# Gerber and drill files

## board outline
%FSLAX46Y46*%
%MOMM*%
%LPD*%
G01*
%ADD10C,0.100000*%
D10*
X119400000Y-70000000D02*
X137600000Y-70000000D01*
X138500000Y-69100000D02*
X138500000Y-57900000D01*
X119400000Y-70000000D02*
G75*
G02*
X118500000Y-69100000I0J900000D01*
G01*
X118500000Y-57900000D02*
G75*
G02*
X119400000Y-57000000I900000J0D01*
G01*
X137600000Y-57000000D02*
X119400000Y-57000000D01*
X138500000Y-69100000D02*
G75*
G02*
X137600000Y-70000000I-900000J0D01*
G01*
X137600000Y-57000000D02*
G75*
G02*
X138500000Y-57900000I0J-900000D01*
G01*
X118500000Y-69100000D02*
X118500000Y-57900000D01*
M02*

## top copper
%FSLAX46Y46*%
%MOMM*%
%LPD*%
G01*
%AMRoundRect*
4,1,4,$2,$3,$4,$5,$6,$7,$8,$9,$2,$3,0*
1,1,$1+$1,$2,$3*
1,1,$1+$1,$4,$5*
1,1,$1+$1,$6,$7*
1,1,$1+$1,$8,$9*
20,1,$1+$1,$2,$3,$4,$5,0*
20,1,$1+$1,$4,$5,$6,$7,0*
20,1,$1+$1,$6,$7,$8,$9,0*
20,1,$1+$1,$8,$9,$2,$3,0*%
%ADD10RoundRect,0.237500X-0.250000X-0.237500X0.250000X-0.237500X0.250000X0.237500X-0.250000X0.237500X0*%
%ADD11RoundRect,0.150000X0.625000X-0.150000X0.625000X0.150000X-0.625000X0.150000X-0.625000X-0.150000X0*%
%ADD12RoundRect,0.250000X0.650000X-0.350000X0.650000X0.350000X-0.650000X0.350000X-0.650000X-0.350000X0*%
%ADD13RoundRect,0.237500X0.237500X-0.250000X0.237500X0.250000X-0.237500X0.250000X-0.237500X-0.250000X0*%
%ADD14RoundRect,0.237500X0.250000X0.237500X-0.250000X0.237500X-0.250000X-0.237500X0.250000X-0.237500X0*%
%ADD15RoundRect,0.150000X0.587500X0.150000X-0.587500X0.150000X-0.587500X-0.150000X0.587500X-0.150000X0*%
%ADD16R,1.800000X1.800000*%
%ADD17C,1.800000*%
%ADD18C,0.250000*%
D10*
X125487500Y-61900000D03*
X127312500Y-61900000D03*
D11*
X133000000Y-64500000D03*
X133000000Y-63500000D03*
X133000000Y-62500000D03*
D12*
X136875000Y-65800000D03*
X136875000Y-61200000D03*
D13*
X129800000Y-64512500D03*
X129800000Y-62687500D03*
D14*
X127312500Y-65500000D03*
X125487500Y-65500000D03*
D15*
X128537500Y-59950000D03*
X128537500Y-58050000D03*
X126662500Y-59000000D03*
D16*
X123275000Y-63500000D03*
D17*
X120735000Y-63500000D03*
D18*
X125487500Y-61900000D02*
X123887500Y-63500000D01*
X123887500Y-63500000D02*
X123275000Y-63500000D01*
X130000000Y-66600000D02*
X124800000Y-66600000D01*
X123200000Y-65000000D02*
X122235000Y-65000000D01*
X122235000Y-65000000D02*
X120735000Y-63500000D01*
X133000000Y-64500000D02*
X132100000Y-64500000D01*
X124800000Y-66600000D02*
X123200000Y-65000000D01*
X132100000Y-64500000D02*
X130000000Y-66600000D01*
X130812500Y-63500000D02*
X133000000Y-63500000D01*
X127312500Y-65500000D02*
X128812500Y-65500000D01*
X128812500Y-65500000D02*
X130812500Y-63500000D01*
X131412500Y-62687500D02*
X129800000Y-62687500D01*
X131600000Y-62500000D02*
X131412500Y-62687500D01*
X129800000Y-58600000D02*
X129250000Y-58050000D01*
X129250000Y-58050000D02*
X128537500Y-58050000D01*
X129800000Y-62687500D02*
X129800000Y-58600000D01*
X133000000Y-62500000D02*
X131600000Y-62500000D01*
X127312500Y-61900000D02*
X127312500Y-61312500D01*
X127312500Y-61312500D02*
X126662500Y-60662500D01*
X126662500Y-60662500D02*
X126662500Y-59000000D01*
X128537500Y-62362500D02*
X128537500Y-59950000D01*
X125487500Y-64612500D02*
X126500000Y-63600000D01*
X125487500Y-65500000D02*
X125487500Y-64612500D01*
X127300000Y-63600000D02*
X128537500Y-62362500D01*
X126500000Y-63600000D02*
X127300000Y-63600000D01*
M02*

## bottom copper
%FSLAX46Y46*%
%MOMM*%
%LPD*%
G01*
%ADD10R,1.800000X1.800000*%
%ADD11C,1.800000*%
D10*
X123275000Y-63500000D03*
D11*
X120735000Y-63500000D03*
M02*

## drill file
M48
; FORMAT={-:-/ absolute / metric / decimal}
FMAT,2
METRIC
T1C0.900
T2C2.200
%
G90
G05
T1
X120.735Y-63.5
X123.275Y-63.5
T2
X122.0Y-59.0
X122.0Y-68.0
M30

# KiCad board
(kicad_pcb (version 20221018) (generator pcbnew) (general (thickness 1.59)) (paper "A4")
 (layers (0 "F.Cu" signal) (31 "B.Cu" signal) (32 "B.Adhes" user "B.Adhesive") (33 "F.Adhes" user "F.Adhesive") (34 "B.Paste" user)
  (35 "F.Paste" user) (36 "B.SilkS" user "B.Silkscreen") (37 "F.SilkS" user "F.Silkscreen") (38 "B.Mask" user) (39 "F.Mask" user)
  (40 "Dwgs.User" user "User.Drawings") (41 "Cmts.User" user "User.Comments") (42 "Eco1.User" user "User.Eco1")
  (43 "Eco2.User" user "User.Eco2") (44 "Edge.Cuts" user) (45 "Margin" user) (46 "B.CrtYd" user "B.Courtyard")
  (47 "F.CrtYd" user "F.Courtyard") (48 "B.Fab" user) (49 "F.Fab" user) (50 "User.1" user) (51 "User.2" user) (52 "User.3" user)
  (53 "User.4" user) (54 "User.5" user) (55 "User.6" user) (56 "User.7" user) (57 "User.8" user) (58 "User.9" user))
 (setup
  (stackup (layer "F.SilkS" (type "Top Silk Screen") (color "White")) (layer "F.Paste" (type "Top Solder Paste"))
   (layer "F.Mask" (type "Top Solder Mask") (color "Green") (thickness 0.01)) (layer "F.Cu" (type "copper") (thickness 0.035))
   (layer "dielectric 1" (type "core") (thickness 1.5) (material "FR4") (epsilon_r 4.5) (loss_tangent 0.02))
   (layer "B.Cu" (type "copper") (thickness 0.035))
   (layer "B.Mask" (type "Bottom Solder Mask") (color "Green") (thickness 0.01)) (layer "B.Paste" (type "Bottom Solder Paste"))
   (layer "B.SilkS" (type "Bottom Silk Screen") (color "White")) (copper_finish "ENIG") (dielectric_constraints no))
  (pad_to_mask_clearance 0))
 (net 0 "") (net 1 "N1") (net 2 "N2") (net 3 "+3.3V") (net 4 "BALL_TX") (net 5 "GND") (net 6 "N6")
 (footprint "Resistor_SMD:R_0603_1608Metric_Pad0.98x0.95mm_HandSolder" (layer "F.Cu") (at 126.4 61.9)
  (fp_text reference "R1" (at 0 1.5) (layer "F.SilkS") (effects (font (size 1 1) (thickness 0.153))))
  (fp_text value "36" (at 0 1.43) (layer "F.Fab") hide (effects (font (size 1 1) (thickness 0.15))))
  (pad "1" smd roundrect (at -0.9125 0) (size 0.975 0.95) (layers "F.Cu" "F.Paste" "F.Mask") (roundrect_rratio 0.25) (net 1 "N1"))
  (pad "2" smd roundrect (at 0.9125 0) (size 0.975 0.95) (layers "F.Cu" "F.Paste" "F.Mask") (roundrect_rratio 0.25) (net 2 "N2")))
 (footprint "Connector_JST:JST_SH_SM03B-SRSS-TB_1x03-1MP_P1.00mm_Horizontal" (layer "F.Cu") (at 135 63.5 90)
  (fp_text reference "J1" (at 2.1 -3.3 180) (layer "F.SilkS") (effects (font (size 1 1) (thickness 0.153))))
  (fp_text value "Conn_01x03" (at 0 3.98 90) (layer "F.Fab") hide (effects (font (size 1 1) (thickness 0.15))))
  (pad "1" smd roundrect (at -1 -2 90) (size 0.6 1.55) (layers "F.Cu" "F.Paste" "F.Mask") (roundrect_rratio 0.25) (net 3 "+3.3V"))
  (pad "2" smd roundrect (at 0 -2 90) (size 0.6 1.55) (layers "F.Cu" "F.Paste" "F.Mask") (roundrect_rratio 0.25) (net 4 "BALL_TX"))
  (pad "3" smd roundrect (at 1 -2 90) (size 0.6 1.55) (layers "F.Cu" "F.Paste" "F.Mask") (roundrect_rratio 0.25) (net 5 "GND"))
  (pad "MP" smd roundrect (at -2.3 1.875 90) (size 1.2 1.8) (layers "F.Cu" "F.Paste" "F.Mask") (roundrect_rratio 0.2083333333))
  (pad "MP" smd roundrect (at 2.3 1.875 90) (size 1.2 1.8) (layers "F.Cu" "F.Paste" "F.Mask") (roundrect_rratio 0.2083333333)))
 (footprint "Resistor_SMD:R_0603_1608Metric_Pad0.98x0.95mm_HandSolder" (layer "F.Cu") (at 129.8 63.6 90)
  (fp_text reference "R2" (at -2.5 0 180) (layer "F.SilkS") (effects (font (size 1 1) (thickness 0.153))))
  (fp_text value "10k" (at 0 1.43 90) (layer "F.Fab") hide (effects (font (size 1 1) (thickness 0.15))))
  (pad "1" smd roundrect (at -0.9125 0 90) (size 0.975 0.95) (layers "F.Cu" "F.Paste" "F.Mask") (roundrect_rratio 0.25) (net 4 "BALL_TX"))
  (pad "2" smd roundrect (at 0.9125 0 90) (size 0.975 0.95) (layers "F.Cu" "F.Paste" "F.Mask") (roundrect_rratio 0.25) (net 5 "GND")))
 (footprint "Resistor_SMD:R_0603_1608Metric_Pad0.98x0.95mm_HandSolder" (layer "F.Cu") (at 126.4 65.5 180)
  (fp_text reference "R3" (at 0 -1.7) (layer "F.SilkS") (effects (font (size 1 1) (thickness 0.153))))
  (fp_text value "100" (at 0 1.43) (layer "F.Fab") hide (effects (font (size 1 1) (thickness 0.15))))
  (pad "1" smd roundrect (at -0.9125 0 180) (size 0.975 0.95) (layers "F.Cu" "F.Paste" "F.Mask") (roundrect_rratio 0.25) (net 4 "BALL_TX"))
  (pad "2" smd roundrect (at 0.9125 0 180) (size 0.975 0.95) (layers "F.Cu" "F.Paste" "F.Mask") (roundrect_rratio 0.25) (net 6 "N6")))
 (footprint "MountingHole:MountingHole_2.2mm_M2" (layer "F.Cu") (at 122 68 -90)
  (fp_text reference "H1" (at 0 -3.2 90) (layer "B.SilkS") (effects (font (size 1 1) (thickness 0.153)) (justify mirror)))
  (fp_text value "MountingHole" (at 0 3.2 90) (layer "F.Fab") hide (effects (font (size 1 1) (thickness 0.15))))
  (pad "" np_thru_hole circle (at 0 0 270) (size 2.2 2.2) (drill 2.2) (layers "*.Cu" "*.Mask")))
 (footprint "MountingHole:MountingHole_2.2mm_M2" (layer "F.Cu") (at 122 59 -90)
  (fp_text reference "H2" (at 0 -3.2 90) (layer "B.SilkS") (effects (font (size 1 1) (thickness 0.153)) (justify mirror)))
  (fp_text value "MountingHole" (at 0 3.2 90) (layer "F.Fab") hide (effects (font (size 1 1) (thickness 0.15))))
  (pad "" np_thru_hole circle (at 0 0 270) (size 2.2 2.2) (drill 2.2) (layers "*.Cu" "*.Mask")))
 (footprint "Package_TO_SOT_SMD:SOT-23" (layer "F.Cu") (at 127.6 59 180)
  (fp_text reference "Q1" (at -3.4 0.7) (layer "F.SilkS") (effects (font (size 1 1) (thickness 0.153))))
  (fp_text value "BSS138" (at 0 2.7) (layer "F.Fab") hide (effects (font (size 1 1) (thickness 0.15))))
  (pad "1" smd roundrect (at -0.9375 -0.95 180) (size 1.475 0.6) (layers "F.Cu" "F.Paste" "F.Mask") (roundrect_rratio 0.25) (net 6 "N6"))
  (pad "2" smd roundrect (at -0.9375 0.95 180) (size 1.475 0.6) (layers "F.Cu" "F.Paste" "F.Mask") (roundrect_rratio 0.25) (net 5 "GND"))
  (pad "3" smd roundrect (at 0.9375 0 180) (size 1.475 0.6) (layers "F.Cu" "F.Paste" "F.Mask") (roundrect_rratio 0.25) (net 2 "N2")))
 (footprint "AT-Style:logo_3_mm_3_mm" (layer "B.Cu") (at 135.5 60.5 180)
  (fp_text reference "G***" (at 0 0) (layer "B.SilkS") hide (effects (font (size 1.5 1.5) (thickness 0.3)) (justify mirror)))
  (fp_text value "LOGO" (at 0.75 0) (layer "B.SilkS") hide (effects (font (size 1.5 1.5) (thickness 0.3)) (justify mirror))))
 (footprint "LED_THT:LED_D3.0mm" (layer "B.Cu") (at 123.275 63.5 180)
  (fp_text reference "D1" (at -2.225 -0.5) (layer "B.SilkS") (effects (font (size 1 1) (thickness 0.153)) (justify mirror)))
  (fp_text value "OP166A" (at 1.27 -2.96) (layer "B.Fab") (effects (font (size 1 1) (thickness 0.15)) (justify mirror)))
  (pad "1" thru_hole rect (at 0 0 180) (size 1.8 1.8) (drill 0.9) (layers "*.Cu" "*.Mask") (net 1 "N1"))
  (pad "2" thru_hole circle (at 2.54 0 180) (size 1.8 1.8) (drill 0.9) (layers "*.Cu" "*.Mask") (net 3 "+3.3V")))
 (gr_line (start 119.4 70) (end 137.6 70) (stroke (width 0.1) (type default)) (layer "Edge.Cuts"))
 (gr_line (start 138.5 69.1) (end 138.5 57.9) (stroke (width 0.1) (type default)) (layer "Edge.Cuts"))
 (gr_arc (start 119.4 70) (mid 118.763604 69.736396) (end 118.5 69.1) (stroke (width 0.1) (type default)) (layer "Edge.Cuts"))
 (gr_arc (start 118.5 57.9) (mid 118.763604 57.263604) (end 119.4 57) (stroke (width 0.1) (type default)) (layer "Edge.Cuts"))
 (gr_line (start 137.6 57) (end 119.4 57) (stroke (width 0.1) (type default)) (layer "Edge.Cuts"))
 (gr_arc (start 138.5 69.1) (mid 138.236396 69.736396) (end 137.6 70) (stroke (width 0.1) (type default)) (layer "Edge.Cuts"))
 (gr_arc (start 137.6 57) (mid 138.236396 57.263604) (end 138.5 57.9) (stroke (width 0.1) (type default)) (layer "Edge.Cuts"))
 (gr_line (start 118.5 69.1) (end 118.5 57.9) (stroke (width 0.1) (type default)) (layer "Edge.Cuts"))
 (segment (start 125.4875 61.9) (end 123.8875 63.5) (width 0.25) (layer "F.Cu") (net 1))
 (segment (start 123.8875 63.5) (end 123.275 63.5) (width 0.25) (layer "F.Cu") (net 1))
 (segment (start 130 66.6) (end 124.8 66.6) (width 0.25) (layer "F.Cu") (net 3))
 (segment (start 123.2 65) (end 122.235 65) (width 0.25) (layer "F.Cu") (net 3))
 (segment (start 122.235 65) (end 120.735 63.5) (width 0.25) (layer "F.Cu") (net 3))
 (segment (start 133 64.5) (end 132.1 64.5) (width 0.25) (layer "F.Cu") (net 3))
 (segment (start 124.8 66.6) (end 123.2 65) (width 0.25) (layer "F.Cu") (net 3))
 (segment (start 132.1 64.5) (end 130 66.6) (width 0.25) (layer "F.Cu") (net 3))
 (segment (start 130.8125 63.5) (end 133 63.5) (width 0.25) (layer "F.Cu") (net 4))
 (segment (start 127.3125 65.5) (end 128.8125 65.5) (width 0.25) (layer "F.Cu") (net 4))
 (segment (start 128.8125 65.5) (end 130.8125 63.5) (width 0.25) (layer "F.Cu") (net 4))
 (segment (start 131.4125 62.6875) (end 129.8 62.6875) (width 0.25) (layer "F.Cu") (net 5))
 (segment (start 131.6 62.5) (end 131.4125 62.6875) (width 0.25) (layer "F.Cu") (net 5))
 (segment (start 129.8 58.6) (end 129.25 58.05) (width 0.25) (layer "F.Cu") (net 5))
 (segment (start 129.25 58.05) (end 128.5375 58.05) (width 0.25) (layer "F.Cu") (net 5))
 (segment (start 129.8 62.6875) (end 129.8 58.6) (width 0.25) (layer "F.Cu") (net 5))
 (segment (start 133 62.5) (end 131.6 62.5) (width 0.25) (layer "F.Cu") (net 5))
 (segment (start 127.3125 61.9) (end 127.3125 61.3125) (width 0.25) (layer "F.Cu") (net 2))
 (segment (start 127.3125 61.3125) (end 126.6625 60.6625) (width 0.25) (layer "F.Cu") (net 2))
 (segment (start 126.6625 60.6625) (end 126.6625 59) (width 0.25) (layer "F.Cu") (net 2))
 (segment (start 128.5375 62.3625) (end 128.5375 59.95) (width 0.25) (layer "F.Cu") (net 6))
 (segment (start 125.4875 64.6125) (end 126.5 63.6) (width 0.25) (layer "F.Cu") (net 6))
 (segment (start 125.4875 65.5) (end 125.4875 64.6125) (width 0.25) (layer "F.Cu") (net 6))
 (segment (start 127.3 63.6) (end 128.5375 62.3625) (width 0.25) (layer "F.Cu") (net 6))
 (segment (start 126.5 63.6) (end 127.3 63.6) (width 0.25) (layer "F.Cu") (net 6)))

